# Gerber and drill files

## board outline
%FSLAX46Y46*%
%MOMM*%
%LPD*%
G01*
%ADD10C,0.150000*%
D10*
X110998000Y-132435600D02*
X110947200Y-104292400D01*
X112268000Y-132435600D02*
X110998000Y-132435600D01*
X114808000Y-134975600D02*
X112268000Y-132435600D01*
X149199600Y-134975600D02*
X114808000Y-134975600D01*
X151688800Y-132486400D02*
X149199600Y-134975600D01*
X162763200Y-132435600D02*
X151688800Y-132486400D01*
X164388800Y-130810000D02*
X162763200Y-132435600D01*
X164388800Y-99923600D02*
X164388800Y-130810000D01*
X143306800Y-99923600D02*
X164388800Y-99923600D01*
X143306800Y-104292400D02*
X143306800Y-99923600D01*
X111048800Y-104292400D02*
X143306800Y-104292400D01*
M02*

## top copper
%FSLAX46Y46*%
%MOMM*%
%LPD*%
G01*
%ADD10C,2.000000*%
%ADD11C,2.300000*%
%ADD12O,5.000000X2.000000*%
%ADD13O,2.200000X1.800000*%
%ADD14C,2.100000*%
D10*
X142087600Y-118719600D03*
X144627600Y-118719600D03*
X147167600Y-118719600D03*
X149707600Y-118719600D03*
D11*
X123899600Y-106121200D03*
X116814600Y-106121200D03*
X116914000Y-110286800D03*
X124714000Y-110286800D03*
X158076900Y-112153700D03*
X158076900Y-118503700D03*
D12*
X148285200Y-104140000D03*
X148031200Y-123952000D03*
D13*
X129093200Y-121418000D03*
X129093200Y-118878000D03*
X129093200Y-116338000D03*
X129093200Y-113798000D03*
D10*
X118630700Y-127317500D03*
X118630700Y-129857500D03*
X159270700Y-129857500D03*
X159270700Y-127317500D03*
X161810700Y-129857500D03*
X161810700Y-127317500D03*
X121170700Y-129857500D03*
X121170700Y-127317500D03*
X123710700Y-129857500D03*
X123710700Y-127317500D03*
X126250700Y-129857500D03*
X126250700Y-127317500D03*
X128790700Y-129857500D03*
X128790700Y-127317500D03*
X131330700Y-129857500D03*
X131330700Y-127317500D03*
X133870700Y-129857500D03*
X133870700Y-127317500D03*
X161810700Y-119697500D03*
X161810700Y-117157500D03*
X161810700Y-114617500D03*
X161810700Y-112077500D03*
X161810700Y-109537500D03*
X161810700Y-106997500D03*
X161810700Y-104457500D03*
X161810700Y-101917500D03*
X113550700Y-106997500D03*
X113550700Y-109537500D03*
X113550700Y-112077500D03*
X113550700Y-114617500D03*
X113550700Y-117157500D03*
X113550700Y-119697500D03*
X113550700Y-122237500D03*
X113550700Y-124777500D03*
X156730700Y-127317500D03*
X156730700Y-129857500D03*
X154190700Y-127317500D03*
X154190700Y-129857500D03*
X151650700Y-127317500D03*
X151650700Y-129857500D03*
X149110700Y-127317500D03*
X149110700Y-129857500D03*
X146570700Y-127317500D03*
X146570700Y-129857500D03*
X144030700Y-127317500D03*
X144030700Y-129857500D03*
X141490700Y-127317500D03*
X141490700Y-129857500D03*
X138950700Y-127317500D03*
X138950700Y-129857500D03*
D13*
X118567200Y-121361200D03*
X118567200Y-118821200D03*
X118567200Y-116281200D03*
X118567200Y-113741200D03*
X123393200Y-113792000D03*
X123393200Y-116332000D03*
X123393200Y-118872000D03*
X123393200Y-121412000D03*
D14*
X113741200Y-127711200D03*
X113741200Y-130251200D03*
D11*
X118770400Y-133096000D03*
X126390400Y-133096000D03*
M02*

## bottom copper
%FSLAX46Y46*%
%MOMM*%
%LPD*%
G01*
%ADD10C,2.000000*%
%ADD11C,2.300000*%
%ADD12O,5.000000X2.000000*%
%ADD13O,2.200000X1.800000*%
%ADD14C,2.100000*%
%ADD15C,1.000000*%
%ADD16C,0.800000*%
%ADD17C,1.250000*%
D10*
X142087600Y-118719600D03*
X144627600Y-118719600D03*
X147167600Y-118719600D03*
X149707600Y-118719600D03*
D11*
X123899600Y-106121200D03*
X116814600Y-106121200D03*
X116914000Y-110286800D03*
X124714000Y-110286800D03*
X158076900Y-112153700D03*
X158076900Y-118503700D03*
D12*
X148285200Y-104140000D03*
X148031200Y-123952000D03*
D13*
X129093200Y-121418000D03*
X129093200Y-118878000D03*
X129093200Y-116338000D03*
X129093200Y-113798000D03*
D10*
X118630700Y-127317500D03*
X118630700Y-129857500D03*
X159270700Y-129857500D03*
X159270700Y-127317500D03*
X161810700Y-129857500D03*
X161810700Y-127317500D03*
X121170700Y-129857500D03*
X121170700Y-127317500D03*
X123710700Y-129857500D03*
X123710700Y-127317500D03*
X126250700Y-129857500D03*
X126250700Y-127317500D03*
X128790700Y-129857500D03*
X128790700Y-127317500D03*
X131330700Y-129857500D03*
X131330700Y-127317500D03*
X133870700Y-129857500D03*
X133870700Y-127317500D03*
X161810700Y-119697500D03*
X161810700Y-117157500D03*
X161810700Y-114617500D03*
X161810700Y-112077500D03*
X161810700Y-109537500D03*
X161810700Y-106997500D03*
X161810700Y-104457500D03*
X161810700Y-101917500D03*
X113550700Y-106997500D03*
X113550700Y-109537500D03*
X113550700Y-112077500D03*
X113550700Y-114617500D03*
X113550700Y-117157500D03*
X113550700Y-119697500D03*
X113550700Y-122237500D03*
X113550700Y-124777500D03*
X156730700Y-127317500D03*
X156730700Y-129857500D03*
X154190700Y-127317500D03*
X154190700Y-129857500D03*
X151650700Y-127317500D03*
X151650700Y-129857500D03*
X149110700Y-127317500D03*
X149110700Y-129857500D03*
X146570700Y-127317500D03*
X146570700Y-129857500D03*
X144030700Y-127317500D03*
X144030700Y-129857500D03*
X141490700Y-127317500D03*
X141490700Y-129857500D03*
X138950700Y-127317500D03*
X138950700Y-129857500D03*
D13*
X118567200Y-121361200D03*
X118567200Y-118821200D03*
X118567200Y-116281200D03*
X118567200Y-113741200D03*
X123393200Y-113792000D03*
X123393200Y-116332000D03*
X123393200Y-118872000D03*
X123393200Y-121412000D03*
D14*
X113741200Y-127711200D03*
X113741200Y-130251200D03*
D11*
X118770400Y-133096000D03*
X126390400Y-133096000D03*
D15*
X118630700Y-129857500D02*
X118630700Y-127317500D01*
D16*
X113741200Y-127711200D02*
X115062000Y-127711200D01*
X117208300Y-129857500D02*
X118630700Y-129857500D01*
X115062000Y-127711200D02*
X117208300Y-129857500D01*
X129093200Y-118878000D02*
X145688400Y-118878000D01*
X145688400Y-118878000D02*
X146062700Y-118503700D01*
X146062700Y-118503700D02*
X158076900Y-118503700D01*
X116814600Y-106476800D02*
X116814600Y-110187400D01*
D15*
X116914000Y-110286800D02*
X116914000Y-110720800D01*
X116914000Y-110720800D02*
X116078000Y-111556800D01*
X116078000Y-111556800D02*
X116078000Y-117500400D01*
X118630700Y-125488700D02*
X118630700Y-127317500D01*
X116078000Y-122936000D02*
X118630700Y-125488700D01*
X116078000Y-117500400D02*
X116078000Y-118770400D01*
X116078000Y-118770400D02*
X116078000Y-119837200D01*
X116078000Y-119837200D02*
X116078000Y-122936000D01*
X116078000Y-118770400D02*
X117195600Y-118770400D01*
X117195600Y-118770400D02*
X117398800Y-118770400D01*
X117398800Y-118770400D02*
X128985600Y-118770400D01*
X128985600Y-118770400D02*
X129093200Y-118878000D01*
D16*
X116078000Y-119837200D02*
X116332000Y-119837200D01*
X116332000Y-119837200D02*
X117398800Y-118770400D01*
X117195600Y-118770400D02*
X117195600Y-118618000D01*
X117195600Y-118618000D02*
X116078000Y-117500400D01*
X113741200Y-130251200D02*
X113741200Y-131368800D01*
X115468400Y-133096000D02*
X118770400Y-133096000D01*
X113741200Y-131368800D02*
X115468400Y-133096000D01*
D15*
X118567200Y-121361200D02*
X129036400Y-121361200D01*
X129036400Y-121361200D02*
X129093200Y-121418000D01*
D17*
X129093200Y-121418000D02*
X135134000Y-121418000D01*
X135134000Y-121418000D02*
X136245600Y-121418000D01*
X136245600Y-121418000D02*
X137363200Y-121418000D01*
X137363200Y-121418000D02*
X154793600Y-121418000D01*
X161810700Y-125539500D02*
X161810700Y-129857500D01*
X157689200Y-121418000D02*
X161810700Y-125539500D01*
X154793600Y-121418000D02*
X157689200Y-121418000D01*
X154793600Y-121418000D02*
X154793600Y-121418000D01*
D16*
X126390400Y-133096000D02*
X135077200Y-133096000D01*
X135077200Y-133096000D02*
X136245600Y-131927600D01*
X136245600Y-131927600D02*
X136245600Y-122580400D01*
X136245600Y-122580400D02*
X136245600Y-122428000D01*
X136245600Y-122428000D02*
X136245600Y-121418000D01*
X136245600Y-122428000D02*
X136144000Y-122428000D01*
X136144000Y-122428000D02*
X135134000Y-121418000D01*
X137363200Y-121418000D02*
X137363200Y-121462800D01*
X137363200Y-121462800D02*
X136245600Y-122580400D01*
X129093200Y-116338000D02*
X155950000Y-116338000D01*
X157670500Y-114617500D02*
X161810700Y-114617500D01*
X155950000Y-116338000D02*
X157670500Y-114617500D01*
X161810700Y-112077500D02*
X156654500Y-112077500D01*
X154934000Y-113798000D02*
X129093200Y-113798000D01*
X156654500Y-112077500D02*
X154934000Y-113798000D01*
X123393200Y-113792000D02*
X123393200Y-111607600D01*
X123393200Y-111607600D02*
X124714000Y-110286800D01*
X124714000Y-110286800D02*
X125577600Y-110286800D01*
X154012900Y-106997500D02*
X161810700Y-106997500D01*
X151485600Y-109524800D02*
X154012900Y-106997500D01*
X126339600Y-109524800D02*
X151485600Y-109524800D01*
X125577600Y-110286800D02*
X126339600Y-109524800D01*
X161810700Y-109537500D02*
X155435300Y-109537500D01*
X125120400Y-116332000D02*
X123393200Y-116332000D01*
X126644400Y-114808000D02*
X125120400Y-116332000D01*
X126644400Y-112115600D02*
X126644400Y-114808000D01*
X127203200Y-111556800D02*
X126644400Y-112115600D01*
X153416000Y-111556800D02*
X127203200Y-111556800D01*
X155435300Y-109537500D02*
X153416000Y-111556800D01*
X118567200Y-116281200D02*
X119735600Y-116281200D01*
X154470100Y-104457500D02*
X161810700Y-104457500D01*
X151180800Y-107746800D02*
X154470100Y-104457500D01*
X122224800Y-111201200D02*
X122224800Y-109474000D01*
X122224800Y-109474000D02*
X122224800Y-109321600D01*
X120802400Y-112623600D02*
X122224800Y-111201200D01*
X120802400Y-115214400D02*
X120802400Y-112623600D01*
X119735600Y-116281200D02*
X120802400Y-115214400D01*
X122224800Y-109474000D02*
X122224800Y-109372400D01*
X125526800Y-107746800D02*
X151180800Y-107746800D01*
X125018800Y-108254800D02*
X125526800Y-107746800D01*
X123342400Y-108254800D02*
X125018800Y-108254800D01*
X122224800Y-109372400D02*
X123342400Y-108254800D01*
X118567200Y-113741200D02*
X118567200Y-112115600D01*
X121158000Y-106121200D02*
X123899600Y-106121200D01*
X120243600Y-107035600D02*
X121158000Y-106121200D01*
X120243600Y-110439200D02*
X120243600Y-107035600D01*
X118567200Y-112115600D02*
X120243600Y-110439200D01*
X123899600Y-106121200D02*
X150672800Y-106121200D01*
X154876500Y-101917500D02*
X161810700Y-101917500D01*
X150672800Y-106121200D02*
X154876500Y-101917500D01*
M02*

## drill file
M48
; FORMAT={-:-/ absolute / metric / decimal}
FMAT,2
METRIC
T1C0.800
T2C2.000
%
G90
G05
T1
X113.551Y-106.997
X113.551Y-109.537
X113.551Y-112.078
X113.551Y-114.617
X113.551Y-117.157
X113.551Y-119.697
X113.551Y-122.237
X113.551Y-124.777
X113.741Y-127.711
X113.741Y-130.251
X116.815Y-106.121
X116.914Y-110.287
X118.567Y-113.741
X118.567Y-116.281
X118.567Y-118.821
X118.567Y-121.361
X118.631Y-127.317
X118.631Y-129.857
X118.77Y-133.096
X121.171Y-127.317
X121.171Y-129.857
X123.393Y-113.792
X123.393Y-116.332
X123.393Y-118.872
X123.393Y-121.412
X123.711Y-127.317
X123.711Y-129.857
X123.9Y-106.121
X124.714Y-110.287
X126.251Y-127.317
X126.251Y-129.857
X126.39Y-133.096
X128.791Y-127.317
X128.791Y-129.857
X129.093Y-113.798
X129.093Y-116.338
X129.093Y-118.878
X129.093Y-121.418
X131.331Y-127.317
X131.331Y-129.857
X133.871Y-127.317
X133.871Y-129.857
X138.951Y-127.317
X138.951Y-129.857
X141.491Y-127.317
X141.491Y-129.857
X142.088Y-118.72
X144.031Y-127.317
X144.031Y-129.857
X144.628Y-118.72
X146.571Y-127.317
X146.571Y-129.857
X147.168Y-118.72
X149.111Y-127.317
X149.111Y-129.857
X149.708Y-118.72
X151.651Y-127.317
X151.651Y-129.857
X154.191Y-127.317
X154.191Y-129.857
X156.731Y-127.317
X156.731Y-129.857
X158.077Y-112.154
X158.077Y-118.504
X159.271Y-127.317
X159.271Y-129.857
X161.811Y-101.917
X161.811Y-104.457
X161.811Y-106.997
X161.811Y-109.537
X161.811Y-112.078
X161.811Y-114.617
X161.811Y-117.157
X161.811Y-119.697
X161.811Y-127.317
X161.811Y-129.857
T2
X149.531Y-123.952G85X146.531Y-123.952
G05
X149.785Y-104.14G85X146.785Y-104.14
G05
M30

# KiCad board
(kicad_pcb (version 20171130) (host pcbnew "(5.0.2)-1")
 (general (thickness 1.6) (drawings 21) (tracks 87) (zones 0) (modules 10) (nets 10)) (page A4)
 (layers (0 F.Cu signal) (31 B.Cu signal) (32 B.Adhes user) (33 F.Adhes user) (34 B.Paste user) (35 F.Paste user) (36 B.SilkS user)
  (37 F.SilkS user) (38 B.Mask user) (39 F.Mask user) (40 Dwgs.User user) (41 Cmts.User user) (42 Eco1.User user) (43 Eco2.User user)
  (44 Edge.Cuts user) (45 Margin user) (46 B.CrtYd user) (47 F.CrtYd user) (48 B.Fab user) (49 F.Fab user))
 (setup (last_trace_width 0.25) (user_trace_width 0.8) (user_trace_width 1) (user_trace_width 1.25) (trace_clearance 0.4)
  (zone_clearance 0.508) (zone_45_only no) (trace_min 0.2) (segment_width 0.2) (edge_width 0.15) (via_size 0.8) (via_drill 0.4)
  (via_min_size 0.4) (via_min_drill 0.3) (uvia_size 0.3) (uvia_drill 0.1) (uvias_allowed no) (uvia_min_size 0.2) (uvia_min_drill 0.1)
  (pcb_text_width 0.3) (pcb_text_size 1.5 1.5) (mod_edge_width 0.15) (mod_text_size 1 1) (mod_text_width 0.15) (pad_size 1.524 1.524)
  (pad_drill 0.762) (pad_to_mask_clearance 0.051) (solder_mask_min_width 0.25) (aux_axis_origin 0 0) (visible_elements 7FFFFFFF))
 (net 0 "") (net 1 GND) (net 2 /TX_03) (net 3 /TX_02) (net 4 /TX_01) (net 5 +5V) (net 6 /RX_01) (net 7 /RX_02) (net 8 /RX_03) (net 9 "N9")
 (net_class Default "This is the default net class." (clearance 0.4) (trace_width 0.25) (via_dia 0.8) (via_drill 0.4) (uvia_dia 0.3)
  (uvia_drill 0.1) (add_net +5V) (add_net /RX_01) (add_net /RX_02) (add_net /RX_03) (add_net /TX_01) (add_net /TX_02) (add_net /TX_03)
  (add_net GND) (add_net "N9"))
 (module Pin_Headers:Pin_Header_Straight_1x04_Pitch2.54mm (layer F.Cu) (at 142.0876 118.7196 90)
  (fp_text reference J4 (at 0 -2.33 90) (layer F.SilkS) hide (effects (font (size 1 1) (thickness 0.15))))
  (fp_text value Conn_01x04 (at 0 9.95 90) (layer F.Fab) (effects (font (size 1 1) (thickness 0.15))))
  (pad 1 thru_hole circle (at 0 0 90) (size 2 2) (drill 0.8) (layers *.Cu *.Mask) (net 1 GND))
  (pad 2 thru_hole circle (at 0 2.54 90) (size 2 2) (drill 0.8) (layers *.Cu *.Mask) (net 1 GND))
  (pad 3 thru_hole circle (at 0 5.08 90) (size 2 2) (drill 0.8) (layers *.Cu *.Mask) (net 1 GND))
  (pad 4 thru_hole circle (at 0 7.62 90) (size 2 2) (drill 0.8) (layers *.Cu *.Mask) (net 1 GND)))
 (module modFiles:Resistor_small (layer F.Cu) (at 123.7996 106.1212 180)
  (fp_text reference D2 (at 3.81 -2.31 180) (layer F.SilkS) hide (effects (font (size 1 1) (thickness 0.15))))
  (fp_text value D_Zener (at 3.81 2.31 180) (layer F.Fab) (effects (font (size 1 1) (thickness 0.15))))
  (pad 1 thru_hole circle (at -0.1 0 180) (size 2.3 2.3) (drill 0.8) (layers *.Cu *.Mask) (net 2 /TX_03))
  (pad 2 thru_hole circle (at 6.985 0 180) (size 2.3 2.3) (drill 0.8) (layers *.Cu *.Mask) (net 1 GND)))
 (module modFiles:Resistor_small (layer F.Cu) (at 124.714 110.2868 180)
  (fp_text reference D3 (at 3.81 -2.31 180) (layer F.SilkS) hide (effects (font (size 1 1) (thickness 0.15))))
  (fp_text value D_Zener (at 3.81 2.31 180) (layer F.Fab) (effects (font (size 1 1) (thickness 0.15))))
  (pad 2 thru_hole circle (at 7.8 0 180) (size 2.3 2.3) (drill 0.8) (layers *.Cu *.Mask) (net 1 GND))
  (pad 1 thru_hole circle (at 0 0 180) (size 2.3 2.3) (drill 0.8) (layers *.Cu *.Mask) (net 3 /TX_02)))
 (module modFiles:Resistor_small (layer F.Cu) (at 162.2044 116.5352 180)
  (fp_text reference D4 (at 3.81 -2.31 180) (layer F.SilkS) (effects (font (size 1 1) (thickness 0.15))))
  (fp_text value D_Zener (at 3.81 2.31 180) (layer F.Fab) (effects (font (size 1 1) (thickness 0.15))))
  (pad 1 thru_hole circle (at 4.1275 4.3815 270) (size 2.3 2.3) (drill 0.8) (layers *.Cu *.Mask) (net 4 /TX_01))
  (pad 2 thru_hole circle (at 4.1275 -1.9685 270) (size 2.3 2.3) (drill 0.8) (layers *.Cu *.Mask) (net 1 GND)))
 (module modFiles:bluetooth (layer F.Cu) (at 136.0932 118.618 180)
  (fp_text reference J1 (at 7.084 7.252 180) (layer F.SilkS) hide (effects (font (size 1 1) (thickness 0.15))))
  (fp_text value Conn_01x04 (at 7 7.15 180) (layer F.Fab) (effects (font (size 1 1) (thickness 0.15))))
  (pad 0 thru_hole oval (at -12.192 14.478 180) (size 5 2) (drill oval 5 2) (layers *.Cu *.Mask))
  (pad 0 thru_hole oval (at -11.938 -5.334 180) (size 5 2) (drill oval 5 2) (layers *.Cu *.Mask))
  (pad 1 thru_hole oval (at 7 -2.8 180) (size 2.2 1.8) (drill 0.8) (layers *.Cu *.Mask) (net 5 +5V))
  (pad 2 thru_hole oval (at 7 -0.26 180) (size 2.2 1.8) (drill 0.8) (layers *.Cu *.Mask) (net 1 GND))
  (pad 3 thru_hole oval (at 7 2.28 180) (size 2.2 1.8) (drill 0.8) (layers *.Cu *.Mask) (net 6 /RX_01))
  (pad 4 thru_hole oval (at 7 4.82 180) (size 2.2 1.8) (drill 0.8) (layers *.Cu *.Mask) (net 4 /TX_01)))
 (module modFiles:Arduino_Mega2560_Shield (layer F.Cu) (at 155.956 60.6552)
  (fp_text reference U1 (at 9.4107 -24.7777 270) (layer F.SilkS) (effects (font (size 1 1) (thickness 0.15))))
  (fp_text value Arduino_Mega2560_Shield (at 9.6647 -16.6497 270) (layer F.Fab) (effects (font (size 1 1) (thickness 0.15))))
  (pad GND1 thru_hole circle (at -37.3253 66.6623 270) (size 2 2) (drill 0.8) (layers *.Cu *.Mask) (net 1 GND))
  (pad GND2 thru_hole circle (at -37.3253 69.2023 270) (size 2 2) (drill 0.8) (layers *.Cu *.Mask) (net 1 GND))
  (pad 23 thru_hole circle (at 3.3147 69.2023 270) (size 2 2) (drill 0.8) (layers *.Cu *.Mask))
  (pad 22 thru_hole circle (at 3.3147 66.6623 270) (size 2 2) (drill 0.8) (layers *.Cu *.Mask))
  (pad 5V1 thru_hole circle (at 5.8547 69.2023 270) (size 2 2) (drill 0.8) (layers *.Cu *.Mask) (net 5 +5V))
  (pad 5V1 thru_hole circle (at 5.8547 66.6623 270) (size 2 2) (drill 0.8) (layers *.Cu *.Mask) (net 5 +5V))
  (pad 53 thru_hole circle (at -34.7853 69.2023 270) (size 2 2) (drill 0.8) (layers *.Cu *.Mask))
  (pad 52 thru_hole circle (at -34.7853 66.6623 270) (size 2 2) (drill 0.8) (layers *.Cu *.Mask))
  (pad 51 thru_hole circle (at -32.2453 69.2023 270) (size 2 2) (drill 0.8) (layers *.Cu *.Mask))
  (pad 50 thru_hole circle (at -32.2453 66.6623 270) (size 2 2) (drill 0.8) (layers *.Cu *.Mask))
  (pad 49 thru_hole circle (at -29.7053 69.2023 270) (size 2 2) (drill 0.8) (layers *.Cu *.Mask))
  (pad 48 thru_hole circle (at -29.7053 66.6623 270) (size 2 2) (drill 0.8) (layers *.Cu *.Mask))
  (pad 47 thru_hole circle (at -27.1653 69.2023 270) (size 2 2) (drill 0.8) (layers *.Cu *.Mask))
  (pad 46 thru_hole circle (at -27.1653 66.6623 270) (size 2 2) (drill 0.8) (layers *.Cu *.Mask))
  (pad 45 thru_hole circle (at -24.6253 69.2023 270) (size 2 2) (drill 0.8) (layers *.Cu *.Mask))
  (pad 44 thru_hole circle (at -24.6253 66.6623 270) (size 2 2) (drill 0.8) (layers *.Cu *.Mask))
  (pad 43 thru_hole circle (at -22.0853 69.2023 270) (size 2 2) (drill 0.8) (layers *.Cu *.Mask))
  (pad 42 thru_hole circle (at -22.0853 66.6623 270) (size 2 2) (drill 0.8) (layers *.Cu *.Mask))
  (pad 21 thru_hole circle (at 5.8547 59.0423 270) (size 2 2) (drill 0.8) (layers *.Cu *.Mask))
  (pad 20 thru_hole circle (at 5.8547 56.5023 270) (size 2 2) (drill 0.8) (layers *.Cu *.Mask))
  (pad 19 thru_hole circle (at 5.8547 53.9623 270) (size 2 2) (drill 0.8) (layers *.Cu *.Mask) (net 6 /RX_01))
  (pad 18 thru_hole circle (at 5.8547 51.4223 270) (size 2 2) (drill 0.8) (layers *.Cu *.Mask) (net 4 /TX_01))
  (pad 17 thru_hole circle (at 5.8547 48.8823 270) (size 2 2) (drill 0.8) (layers *.Cu *.Mask) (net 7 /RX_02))
  (pad 16 thru_hole circle (at 5.8547 46.3423 270) (size 2 2) (drill 0.8) (layers *.Cu *.Mask) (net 3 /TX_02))
  (pad 15 thru_hole circle (at 5.8547 43.8023 270) (size 2 2) (drill 0.8) (layers *.Cu *.Mask) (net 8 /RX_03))
  (pad 14 thru_hole circle (at 5.8547 41.2623 270) (size 2 2) (drill 0.8) (layers *.Cu *.Mask) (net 2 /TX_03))
  (pad A8 thru_hole circle (at -42.4053 46.3423 270) (size 2 2) (drill 0.8) (layers *.Cu *.Mask))
  (pad A9 thru_hole circle (at -42.4053 48.8823 270) (size 2 2) (drill 0.8) (layers *.Cu *.Mask))
  (pad A10 thru_hole circle (at -42.4053 51.4223 270) (size 2 2) (drill 0.8) (layers *.Cu *.Mask))
  (pad A11 thru_hole circle (at -42.4053 53.9623 270) (size 2 2) (drill 0.8) (layers *.Cu *.Mask))
  (pad A12 thru_hole circle (at -42.4053 56.5023 270) (size 2 2) (drill 0.8) (layers *.Cu *.Mask))
  (pad A13 thru_hole circle (at -42.4053 59.0423 270) (size 2 2) (drill 0.8) (layers *.Cu *.Mask))
  (pad A14 thru_hole circle (at -42.4053 61.5823 270) (size 2 2) (drill 0.8) (layers *.Cu *.Mask))
  (pad A15 thru_hole circle (at -42.4053 64.1223 270) (size 2 2) (drill 0.8) (layers *.Cu *.Mask))
  (pad 24 thru_hole circle (at 0.7747 66.6623 270) (size 2 2) (drill 0.8) (layers *.Cu *.Mask))
  (pad 25 thru_hole circle (at 0.7747 69.2023 270) (size 2 2) (drill 0.8) (layers *.Cu *.Mask))
  (pad 26 thru_hole circle (at -1.7653 66.6623 270) (size 2 2) (drill 0.8) (layers *.Cu *.Mask))
  (pad 27 thru_hole circle (at -1.7653 69.2023 270) (size 2 2) (drill 0.8) (layers *.Cu *.Mask))
  (pad 28 thru_hole circle (at -4.3053 66.6623 270) (size 2 2) (drill 0.8) (layers *.Cu *.Mask))
  (pad 29 thru_hole circle (at -4.3053 69.2023 270) (size 2 2) (drill 0.8) (layers *.Cu *.Mask))
  (pad 30 thru_hole circle (at -6.8453 66.6623 270) (size 2 2) (drill 0.8) (layers *.Cu *.Mask))
  (pad 31 thru_hole circle (at -6.8453 69.2023 270) (size 2 2) (drill 0.8) (layers *.Cu *.Mask))
  (pad 32 thru_hole circle (at -9.3853 66.6623 270) (size 2 2) (drill 0.8) (layers *.Cu *.Mask))
  (pad 33 thru_hole circle (at -9.3853 69.2023 270) (size 2 2) (drill 0.8) (layers *.Cu *.Mask))
  (pad 34 thru_hole circle (at -11.9253 66.6623 270) (size 2 2) (drill 0.8) (layers *.Cu *.Mask))
  (pad 35 thru_hole circle (at -11.9253 69.2023 270) (size 2 2) (drill 0.8) (layers *.Cu *.Mask))
  (pad 36 thru_hole circle (at -14.4653 66.6623 270) (size 2 2) (drill 0.8) (layers *.Cu *.Mask))
  (pad 37 thru_hole circle (at -14.4653 69.2023 270) (size 2 2) (drill 0.8) (layers *.Cu *.Mask))
  (pad 38 thru_hole circle (at -17.0053 66.6623 270) (size 2 2) (drill 0.8) (layers *.Cu *.Mask))
  (pad 39 thru_hole circle (at -17.0053 69.2023 270) (size 2 2) (drill 0.8) (layers *.Cu *.Mask)))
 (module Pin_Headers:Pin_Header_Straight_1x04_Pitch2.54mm (layer F.Cu) (at 118.5672 121.3612 180)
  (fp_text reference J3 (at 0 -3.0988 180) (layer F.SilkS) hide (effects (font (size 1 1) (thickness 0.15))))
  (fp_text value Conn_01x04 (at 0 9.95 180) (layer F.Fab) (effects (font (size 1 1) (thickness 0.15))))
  (pad 1 thru_hole oval (at 0 0 180) (size 2.2 1.8) (drill 0.8) (layers *.Cu *.Mask) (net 5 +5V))
  (pad 2 thru_hole oval (at 0 2.54 180) (size 2.2 1.8) (drill 0.8) (layers *.Cu *.Mask) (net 1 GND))
  (pad 3 thru_hole oval (at 0 5.08 180) (size 2.2 1.8) (drill 0.8) (layers *.Cu *.Mask) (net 8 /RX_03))
  (pad 4 thru_hole oval (at 0 7.62 180) (size 2.2 1.8) (drill 0.8) (layers *.Cu *.Mask) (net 2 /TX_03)))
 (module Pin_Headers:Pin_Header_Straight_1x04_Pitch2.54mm (layer F.Cu) (at 123.3932 121.412 180)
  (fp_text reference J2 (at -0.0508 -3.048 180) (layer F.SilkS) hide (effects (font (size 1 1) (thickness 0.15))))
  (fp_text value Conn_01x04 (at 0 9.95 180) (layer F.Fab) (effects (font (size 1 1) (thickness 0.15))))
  (pad 4 thru_hole oval (at 0 7.62 180) (size 2.2 1.8) (drill 0.8) (layers *.Cu *.Mask) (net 3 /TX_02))
  (pad 3 thru_hole oval (at 0 5.08 180) (size 2.2 1.8) (drill 0.8) (layers *.Cu *.Mask) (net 7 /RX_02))
  (pad 2 thru_hole oval (at 0 2.54 180) (size 2.2 1.8) (drill 0.8) (layers *.Cu *.Mask) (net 1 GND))
  (pad 1 thru_hole oval (at 0 0 180) (size 2.2 1.8) (drill 0.8) (layers *.Cu *.Mask) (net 5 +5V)))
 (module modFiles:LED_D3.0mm (layer F.Cu) (at 113.7412 127.7112 270)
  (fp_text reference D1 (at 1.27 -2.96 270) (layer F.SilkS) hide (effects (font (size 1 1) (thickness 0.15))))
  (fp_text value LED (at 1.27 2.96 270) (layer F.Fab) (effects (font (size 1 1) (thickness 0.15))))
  (pad 1 thru_hole circle (at 0 0 270) (size 2.1 2.1) (drill 0.8) (layers *.Cu *.Mask) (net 1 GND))
  (pad 2 thru_hole circle (at 2.54 0 270) (size 2.1 2.1) (drill 0.8) (layers *.Cu *.Mask) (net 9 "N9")))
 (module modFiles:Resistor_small (layer F.Cu) (at 118.7704 133.096)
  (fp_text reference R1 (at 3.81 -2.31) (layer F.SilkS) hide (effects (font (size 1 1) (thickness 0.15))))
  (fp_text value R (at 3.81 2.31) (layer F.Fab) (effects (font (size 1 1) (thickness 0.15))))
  (pad 1 thru_hole circle (at 0 0) (size 2.3 2.3) (drill 0.8) (layers *.Cu *.Mask) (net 9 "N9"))
  (pad 2 thru_hole circle (at 7.62 0) (size 2.3 2.3) (drill 0.8) (layers *.Cu *.Mask) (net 5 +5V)))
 (gr_line (start 110.998 132.4356) (end 110.9472 104.2924) (angle 90) (layer Edge.Cuts) (width 0.15))
 (gr_line (start 112.268 132.4356) (end 110.998 132.4356) (angle 90) (layer Edge.Cuts) (width 0.15))
 (gr_line (start 114.808 134.9756) (end 112.268 132.4356) (angle 90) (layer Edge.Cuts) (width 0.15))
 (gr_line (start 149.1996 134.9756) (end 114.808 134.9756) (angle 90) (layer Edge.Cuts) (width 0.15))
 (gr_line (start 151.6888 132.4864) (end 149.1996 134.9756) (angle 90) (layer Edge.Cuts) (width 0.15))
 (gr_line (start 162.7632 132.4356) (end 151.6888 132.4864) (angle 90) (layer Edge.Cuts) (width 0.15))
 (gr_line (start 164.3888 130.81) (end 162.7632 132.4356) (angle 90) (layer Edge.Cuts) (width 0.15))
 (gr_line (start 164.3888 99.9236) (end 164.3888 130.81) (angle 90) (layer Edge.Cuts) (width 0.15))
 (gr_line (start 143.3068 99.9236) (end 164.3888 99.9236) (angle 90) (layer Edge.Cuts) (width 0.15))
 (gr_line (start 143.3068 104.2924) (end 143.3068 99.9236) (angle 90) (layer Edge.Cuts) (width 0.15))
 (gr_line (start 111.0488 104.2924) (end 143.3068 104.2924) (angle 90) (layer Edge.Cuts) (width 0.15))
 (segment (start 118.6307 129.8575) (end 118.6307 127.3175) (width 1) (layer B.Cu) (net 1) (status C00000))
 (segment (start 113.7412 127.7112) (end 115.062 127.7112) (width 0.8) (layer B.Cu) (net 1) (status 400000))
 (segment (start 117.2083 129.8575) (end 118.6307 129.8575) (width 0.8) (layer B.Cu) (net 1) (status 800000))
 (segment (start 115.062 127.7112) (end 117.2083 129.8575) (width 0.8) (layer B.Cu) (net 1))
 (segment (start 129.0932 118.878) (end 145.6884 118.878) (width 0.8) (layer B.Cu) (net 1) (status 400000))
 (segment (start 145.6884 118.878) (end 146.0627 118.5037) (width 0.8) (layer B.Cu) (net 1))
 (segment (start 146.0627 118.5037) (end 158.0769 118.5037) (width 0.8) (layer B.Cu) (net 1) (status 800000))
 (segment (start 116.8146 106.4768) (end 116.8146 110.1874) (width 0.8) (layer B.Cu) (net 1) (status C00000))
 (segment (start 116.914 110.2868) (end 116.914 110.7208) (width 1) (layer B.Cu) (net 1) (status C00000))
 (segment (start 116.914 110.7208) (end 116.078 111.5568) (width 1) (layer B.Cu) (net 1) (status 400000))
 (segment (start 116.078 111.5568) (end 116.078 117.5004) (width 1) (layer B.Cu) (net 1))
 (segment (start 118.6307 125.4887) (end 118.6307 127.3175) (width 1) (layer B.Cu) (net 1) (status 800000))
 (segment (start 116.078 122.936) (end 118.6307 125.4887) (width 1) (layer B.Cu) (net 1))
 (segment (start 116.078 117.5004) (end 116.078 118.7704) (width 1) (layer B.Cu) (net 1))
 (segment (start 116.078 118.7704) (end 116.078 119.8372) (width 1) (layer B.Cu) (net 1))
 (segment (start 116.078 119.8372) (end 116.078 122.936) (width 1) (layer B.Cu) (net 1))
 (segment (start 116.078 118.7704) (end 117.1956 118.7704) (width 1) (layer B.Cu) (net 1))
 (segment (start 117.1956 118.7704) (end 117.3988 118.7704) (width 1) (layer B.Cu) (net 1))
 (segment (start 117.3988 118.7704) (end 128.9856 118.7704) (width 1) (layer B.Cu) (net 1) (status 800000))
 (segment (start 128.9856 118.7704) (end 129.0932 118.878) (width 1) (layer B.Cu) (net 1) (status C00000))
 (segment (start 116.078 119.8372) (end 116.332 119.8372) (width 0.8) (layer B.Cu) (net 1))
 (segment (start 116.332 119.8372) (end 117.3988 118.7704) (width 0.8) (layer B.Cu) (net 1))
 (segment (start 117.1956 118.7704) (end 117.1956 118.618) (width 0.8) (layer B.Cu) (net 1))
 (segment (start 117.1956 118.618) (end 116.078 117.5004) (width 0.8) (layer B.Cu) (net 1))
 (segment (start 113.7412 130.2512) (end 113.7412 131.3688) (width 0.8) (layer B.Cu) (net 9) (status 400000))
 (segment (start 115.4684 133.096) (end 118.7704 133.096) (width 0.8) (layer B.Cu) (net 9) (status 800000))
 (segment (start 113.7412 131.3688) (end 115.4684 133.096) (width 0.8) (layer B.Cu) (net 9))
 (segment (start 118.5672 121.3612) (end 129.0364 121.3612) (width 1) (layer B.Cu) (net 5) (status C00000))
 (segment (start 129.0364 121.3612) (end 129.0932 121.418) (width 1) (layer B.Cu) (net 5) (status C00000))
 (segment (start 129.0932 121.418) (end 135.134 121.418) (width 1.25) (layer B.Cu) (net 5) (status 400000))
 (segment (start 135.134 121.418) (end 136.2456 121.418) (width 1.25) (layer B.Cu) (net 5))
 (segment (start 136.2456 121.418) (end 137.3632 121.418) (width 1.25) (layer B.Cu) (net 5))
 (segment (start 137.3632 121.418) (end 154.7936 121.418) (width 1.25) (layer B.Cu) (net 5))
 (segment (start 161.8107 125.5395) (end 161.8107 129.8575) (width 1.25) (layer B.Cu) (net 5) (status 800000))
 (segment (start 157.6892 121.418) (end 161.8107 125.5395) (width 1.25) (layer B.Cu) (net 5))
 (segment (start 154.7936 121.418) (end 157.6892 121.418) (width 1.25) (layer B.Cu) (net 5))
 (segment (start 154.7936 121.418) (end 154.7936 121.418) (width 1.25) (layer B.Cu) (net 5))
 (segment (start 126.3904 133.096) (end 135.0772 133.096) (width 0.8) (layer B.Cu) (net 5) (status 400000))
 (segment (start 135.0772 133.096) (end 136.2456 131.9276) (width 0.8) (layer B.Cu) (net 5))
 (segment (start 136.2456 131.9276) (end 136.2456 122.5804) (width 0.8) (layer B.Cu) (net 5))
 (segment (start 136.2456 122.5804) (end 136.2456 122.428) (width 0.8) (layer B.Cu) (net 5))
 (segment (start 136.2456 122.428) (end 136.2456 121.418) (width 0.8) (layer B.Cu) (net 5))
 (segment (start 136.2456 122.428) (end 136.144 122.428) (width 0.8) (layer B.Cu) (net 5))
 (segment (start 136.144 122.428) (end 135.134 121.418) (width 0.8) (layer B.Cu) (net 5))
 (segment (start 137.3632 121.418) (end 137.3632 121.4628) (width 0.8) (layer B.Cu) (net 5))
 (segment (start 137.3632 121.4628) (end 136.2456 122.5804) (width 0.8) (layer B.Cu) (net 5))
 (segment (start 129.0932 116.338) (end 155.95 116.338) (width 0.8) (layer B.Cu) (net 6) (status 400000))
 (segment (start 157.6705 114.6175) (end 161.8107 114.6175) (width 0.8) (layer B.Cu) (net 6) (status 800000))
 (segment (start 155.95 116.338) (end 157.6705 114.6175) (width 0.8) (layer B.Cu) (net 6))
 (segment (start 161.8107 112.0775) (end 156.6545 112.0775) (width 0.8) (layer B.Cu) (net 4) (status 400000))
 (segment (start 154.934 113.798) (end 129.0932 113.798) (width 0.8) (layer B.Cu) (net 4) (status 800000))
 (segment (start 156.6545 112.0775) (end 154.934 113.798) (width 0.8) (layer B.Cu) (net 4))
 (segment (start 123.3932 113.792) (end 123.3932 111.6076) (width 0.8) (layer B.Cu) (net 3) (status 400000))
 (segment (start 123.3932 111.6076) (end 124.714 110.2868) (width 0.8) (layer B.Cu) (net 3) (status 800000))
 (segment (start 124.714 110.2868) (end 125.5776 110.2868) (width 0.8) (layer B.Cu) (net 3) (status C00000))
 (segment (start 154.0129 106.9975) (end 161.8107 106.9975) (width 0.8) (layer B.Cu) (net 3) (status 800000))
 (segment (start 151.4856 109.5248) (end 154.0129 106.9975) (width 0.8) (layer B.Cu) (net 3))
 (segment (start 126.3396 109.5248) (end 151.4856 109.5248) (width 0.8) (layer B.Cu) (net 3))
 (segment (start 125.5776 110.2868) (end 126.3396 109.5248) (width 0.8) (layer B.Cu) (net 3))
 (segment (start 161.8107 109.5375) (end 155.4353 109.5375) (width 0.8) (layer B.Cu) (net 7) (status 400000))
 (segment (start 125.1204 116.332) (end 123.3932 116.332) (width 0.8) (layer B.Cu) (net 7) (status 800000))
 (segment (start 126.6444 114.808) (end 125.1204 116.332) (width 0.8) (layer B.Cu) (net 7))
 (segment (start 126.6444 112.1156) (end 126.6444 114.808) (width 0.8) (layer B.Cu) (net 7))
 (segment (start 127.2032 111.5568) (end 126.6444 112.1156) (width 0.8) (layer B.Cu) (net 7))
 (segment (start 153.416 111.5568) (end 127.2032 111.5568) (width 0.8) (layer B.Cu) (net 7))
 (segment (start 155.4353 109.5375) (end 153.416 111.5568) (width 0.8) (layer B.Cu) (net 7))
 (segment (start 118.5672 116.2812) (end 119.7356 116.2812) (width 0.8) (layer B.Cu) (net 8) (status 400000))
 (segment (start 154.4701 104.4575) (end 161.8107 104.4575) (width 0.8) (layer B.Cu) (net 8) (status 800000))
 (segment (start 151.1808 107.7468) (end 154.4701 104.4575) (width 0.8) (layer B.Cu) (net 8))
 (segment (start 122.2248 111.2012) (end 122.2248 109.474) (width 0.8) (layer B.Cu) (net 8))
 (segment (start 122.2248 109.474) (end 122.2248 109.3216) (width 0.8) (layer B.Cu) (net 8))
 (segment (start 120.8024 112.6236) (end 122.2248 111.2012) (width 0.8) (layer B.Cu) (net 8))
 (segment (start 120.8024 115.2144) (end 120.8024 112.6236) (width 0.8) (layer B.Cu) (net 8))
 (segment (start 119.7356 116.2812) (end 120.8024 115.2144) (width 0.8) (layer B.Cu) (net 8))
 (segment (start 122.2248 109.474) (end 122.2248 109.3724) (width 0.8) (layer B.Cu) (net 8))
 (segment (start 125.5268 107.7468) (end 151.1808 107.7468) (width 0.8) (layer B.Cu) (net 8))
 (segment (start 125.0188 108.2548) (end 125.5268 107.7468) (width 0.8) (layer B.Cu) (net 8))
 (segment (start 123.3424 108.2548) (end 125.0188 108.2548) (width 0.8) (layer B.Cu) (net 8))
 (segment (start 122.2248 109.3724) (end 123.3424 108.2548) (width 0.8) (layer B.Cu) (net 8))
 (segment (start 118.5672 113.7412) (end 118.5672 112.1156) (width 0.8) (layer B.Cu) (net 2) (status 400000))
 (segment (start 121.158 106.1212) (end 123.8996 106.1212) (width 0.8) (layer B.Cu) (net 2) (status 800000))
 (segment (start 120.2436 107.0356) (end 121.158 106.1212) (width 0.8) (layer B.Cu) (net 2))
 (segment (start 120.2436 110.4392) (end 120.2436 107.0356) (width 0.8) (layer B.Cu) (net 2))
 (segment (start 118.5672 112.1156) (end 120.2436 110.4392) (width 0.8) (layer B.Cu) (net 2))
 (segment (start 123.8996 106.1212) (end 150.6728 106.1212) (width 0.8) (layer B.Cu) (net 2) (status 400000))
 (segment (start 154.8765 101.9175) (end 161.8107 101.9175) (width 0.8) (layer B.Cu) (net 2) (status 800000))
 (segment (start 150.6728 106.1212) (end 154.8765 101.9175) (width 0.8) (layer B.Cu) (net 2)))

